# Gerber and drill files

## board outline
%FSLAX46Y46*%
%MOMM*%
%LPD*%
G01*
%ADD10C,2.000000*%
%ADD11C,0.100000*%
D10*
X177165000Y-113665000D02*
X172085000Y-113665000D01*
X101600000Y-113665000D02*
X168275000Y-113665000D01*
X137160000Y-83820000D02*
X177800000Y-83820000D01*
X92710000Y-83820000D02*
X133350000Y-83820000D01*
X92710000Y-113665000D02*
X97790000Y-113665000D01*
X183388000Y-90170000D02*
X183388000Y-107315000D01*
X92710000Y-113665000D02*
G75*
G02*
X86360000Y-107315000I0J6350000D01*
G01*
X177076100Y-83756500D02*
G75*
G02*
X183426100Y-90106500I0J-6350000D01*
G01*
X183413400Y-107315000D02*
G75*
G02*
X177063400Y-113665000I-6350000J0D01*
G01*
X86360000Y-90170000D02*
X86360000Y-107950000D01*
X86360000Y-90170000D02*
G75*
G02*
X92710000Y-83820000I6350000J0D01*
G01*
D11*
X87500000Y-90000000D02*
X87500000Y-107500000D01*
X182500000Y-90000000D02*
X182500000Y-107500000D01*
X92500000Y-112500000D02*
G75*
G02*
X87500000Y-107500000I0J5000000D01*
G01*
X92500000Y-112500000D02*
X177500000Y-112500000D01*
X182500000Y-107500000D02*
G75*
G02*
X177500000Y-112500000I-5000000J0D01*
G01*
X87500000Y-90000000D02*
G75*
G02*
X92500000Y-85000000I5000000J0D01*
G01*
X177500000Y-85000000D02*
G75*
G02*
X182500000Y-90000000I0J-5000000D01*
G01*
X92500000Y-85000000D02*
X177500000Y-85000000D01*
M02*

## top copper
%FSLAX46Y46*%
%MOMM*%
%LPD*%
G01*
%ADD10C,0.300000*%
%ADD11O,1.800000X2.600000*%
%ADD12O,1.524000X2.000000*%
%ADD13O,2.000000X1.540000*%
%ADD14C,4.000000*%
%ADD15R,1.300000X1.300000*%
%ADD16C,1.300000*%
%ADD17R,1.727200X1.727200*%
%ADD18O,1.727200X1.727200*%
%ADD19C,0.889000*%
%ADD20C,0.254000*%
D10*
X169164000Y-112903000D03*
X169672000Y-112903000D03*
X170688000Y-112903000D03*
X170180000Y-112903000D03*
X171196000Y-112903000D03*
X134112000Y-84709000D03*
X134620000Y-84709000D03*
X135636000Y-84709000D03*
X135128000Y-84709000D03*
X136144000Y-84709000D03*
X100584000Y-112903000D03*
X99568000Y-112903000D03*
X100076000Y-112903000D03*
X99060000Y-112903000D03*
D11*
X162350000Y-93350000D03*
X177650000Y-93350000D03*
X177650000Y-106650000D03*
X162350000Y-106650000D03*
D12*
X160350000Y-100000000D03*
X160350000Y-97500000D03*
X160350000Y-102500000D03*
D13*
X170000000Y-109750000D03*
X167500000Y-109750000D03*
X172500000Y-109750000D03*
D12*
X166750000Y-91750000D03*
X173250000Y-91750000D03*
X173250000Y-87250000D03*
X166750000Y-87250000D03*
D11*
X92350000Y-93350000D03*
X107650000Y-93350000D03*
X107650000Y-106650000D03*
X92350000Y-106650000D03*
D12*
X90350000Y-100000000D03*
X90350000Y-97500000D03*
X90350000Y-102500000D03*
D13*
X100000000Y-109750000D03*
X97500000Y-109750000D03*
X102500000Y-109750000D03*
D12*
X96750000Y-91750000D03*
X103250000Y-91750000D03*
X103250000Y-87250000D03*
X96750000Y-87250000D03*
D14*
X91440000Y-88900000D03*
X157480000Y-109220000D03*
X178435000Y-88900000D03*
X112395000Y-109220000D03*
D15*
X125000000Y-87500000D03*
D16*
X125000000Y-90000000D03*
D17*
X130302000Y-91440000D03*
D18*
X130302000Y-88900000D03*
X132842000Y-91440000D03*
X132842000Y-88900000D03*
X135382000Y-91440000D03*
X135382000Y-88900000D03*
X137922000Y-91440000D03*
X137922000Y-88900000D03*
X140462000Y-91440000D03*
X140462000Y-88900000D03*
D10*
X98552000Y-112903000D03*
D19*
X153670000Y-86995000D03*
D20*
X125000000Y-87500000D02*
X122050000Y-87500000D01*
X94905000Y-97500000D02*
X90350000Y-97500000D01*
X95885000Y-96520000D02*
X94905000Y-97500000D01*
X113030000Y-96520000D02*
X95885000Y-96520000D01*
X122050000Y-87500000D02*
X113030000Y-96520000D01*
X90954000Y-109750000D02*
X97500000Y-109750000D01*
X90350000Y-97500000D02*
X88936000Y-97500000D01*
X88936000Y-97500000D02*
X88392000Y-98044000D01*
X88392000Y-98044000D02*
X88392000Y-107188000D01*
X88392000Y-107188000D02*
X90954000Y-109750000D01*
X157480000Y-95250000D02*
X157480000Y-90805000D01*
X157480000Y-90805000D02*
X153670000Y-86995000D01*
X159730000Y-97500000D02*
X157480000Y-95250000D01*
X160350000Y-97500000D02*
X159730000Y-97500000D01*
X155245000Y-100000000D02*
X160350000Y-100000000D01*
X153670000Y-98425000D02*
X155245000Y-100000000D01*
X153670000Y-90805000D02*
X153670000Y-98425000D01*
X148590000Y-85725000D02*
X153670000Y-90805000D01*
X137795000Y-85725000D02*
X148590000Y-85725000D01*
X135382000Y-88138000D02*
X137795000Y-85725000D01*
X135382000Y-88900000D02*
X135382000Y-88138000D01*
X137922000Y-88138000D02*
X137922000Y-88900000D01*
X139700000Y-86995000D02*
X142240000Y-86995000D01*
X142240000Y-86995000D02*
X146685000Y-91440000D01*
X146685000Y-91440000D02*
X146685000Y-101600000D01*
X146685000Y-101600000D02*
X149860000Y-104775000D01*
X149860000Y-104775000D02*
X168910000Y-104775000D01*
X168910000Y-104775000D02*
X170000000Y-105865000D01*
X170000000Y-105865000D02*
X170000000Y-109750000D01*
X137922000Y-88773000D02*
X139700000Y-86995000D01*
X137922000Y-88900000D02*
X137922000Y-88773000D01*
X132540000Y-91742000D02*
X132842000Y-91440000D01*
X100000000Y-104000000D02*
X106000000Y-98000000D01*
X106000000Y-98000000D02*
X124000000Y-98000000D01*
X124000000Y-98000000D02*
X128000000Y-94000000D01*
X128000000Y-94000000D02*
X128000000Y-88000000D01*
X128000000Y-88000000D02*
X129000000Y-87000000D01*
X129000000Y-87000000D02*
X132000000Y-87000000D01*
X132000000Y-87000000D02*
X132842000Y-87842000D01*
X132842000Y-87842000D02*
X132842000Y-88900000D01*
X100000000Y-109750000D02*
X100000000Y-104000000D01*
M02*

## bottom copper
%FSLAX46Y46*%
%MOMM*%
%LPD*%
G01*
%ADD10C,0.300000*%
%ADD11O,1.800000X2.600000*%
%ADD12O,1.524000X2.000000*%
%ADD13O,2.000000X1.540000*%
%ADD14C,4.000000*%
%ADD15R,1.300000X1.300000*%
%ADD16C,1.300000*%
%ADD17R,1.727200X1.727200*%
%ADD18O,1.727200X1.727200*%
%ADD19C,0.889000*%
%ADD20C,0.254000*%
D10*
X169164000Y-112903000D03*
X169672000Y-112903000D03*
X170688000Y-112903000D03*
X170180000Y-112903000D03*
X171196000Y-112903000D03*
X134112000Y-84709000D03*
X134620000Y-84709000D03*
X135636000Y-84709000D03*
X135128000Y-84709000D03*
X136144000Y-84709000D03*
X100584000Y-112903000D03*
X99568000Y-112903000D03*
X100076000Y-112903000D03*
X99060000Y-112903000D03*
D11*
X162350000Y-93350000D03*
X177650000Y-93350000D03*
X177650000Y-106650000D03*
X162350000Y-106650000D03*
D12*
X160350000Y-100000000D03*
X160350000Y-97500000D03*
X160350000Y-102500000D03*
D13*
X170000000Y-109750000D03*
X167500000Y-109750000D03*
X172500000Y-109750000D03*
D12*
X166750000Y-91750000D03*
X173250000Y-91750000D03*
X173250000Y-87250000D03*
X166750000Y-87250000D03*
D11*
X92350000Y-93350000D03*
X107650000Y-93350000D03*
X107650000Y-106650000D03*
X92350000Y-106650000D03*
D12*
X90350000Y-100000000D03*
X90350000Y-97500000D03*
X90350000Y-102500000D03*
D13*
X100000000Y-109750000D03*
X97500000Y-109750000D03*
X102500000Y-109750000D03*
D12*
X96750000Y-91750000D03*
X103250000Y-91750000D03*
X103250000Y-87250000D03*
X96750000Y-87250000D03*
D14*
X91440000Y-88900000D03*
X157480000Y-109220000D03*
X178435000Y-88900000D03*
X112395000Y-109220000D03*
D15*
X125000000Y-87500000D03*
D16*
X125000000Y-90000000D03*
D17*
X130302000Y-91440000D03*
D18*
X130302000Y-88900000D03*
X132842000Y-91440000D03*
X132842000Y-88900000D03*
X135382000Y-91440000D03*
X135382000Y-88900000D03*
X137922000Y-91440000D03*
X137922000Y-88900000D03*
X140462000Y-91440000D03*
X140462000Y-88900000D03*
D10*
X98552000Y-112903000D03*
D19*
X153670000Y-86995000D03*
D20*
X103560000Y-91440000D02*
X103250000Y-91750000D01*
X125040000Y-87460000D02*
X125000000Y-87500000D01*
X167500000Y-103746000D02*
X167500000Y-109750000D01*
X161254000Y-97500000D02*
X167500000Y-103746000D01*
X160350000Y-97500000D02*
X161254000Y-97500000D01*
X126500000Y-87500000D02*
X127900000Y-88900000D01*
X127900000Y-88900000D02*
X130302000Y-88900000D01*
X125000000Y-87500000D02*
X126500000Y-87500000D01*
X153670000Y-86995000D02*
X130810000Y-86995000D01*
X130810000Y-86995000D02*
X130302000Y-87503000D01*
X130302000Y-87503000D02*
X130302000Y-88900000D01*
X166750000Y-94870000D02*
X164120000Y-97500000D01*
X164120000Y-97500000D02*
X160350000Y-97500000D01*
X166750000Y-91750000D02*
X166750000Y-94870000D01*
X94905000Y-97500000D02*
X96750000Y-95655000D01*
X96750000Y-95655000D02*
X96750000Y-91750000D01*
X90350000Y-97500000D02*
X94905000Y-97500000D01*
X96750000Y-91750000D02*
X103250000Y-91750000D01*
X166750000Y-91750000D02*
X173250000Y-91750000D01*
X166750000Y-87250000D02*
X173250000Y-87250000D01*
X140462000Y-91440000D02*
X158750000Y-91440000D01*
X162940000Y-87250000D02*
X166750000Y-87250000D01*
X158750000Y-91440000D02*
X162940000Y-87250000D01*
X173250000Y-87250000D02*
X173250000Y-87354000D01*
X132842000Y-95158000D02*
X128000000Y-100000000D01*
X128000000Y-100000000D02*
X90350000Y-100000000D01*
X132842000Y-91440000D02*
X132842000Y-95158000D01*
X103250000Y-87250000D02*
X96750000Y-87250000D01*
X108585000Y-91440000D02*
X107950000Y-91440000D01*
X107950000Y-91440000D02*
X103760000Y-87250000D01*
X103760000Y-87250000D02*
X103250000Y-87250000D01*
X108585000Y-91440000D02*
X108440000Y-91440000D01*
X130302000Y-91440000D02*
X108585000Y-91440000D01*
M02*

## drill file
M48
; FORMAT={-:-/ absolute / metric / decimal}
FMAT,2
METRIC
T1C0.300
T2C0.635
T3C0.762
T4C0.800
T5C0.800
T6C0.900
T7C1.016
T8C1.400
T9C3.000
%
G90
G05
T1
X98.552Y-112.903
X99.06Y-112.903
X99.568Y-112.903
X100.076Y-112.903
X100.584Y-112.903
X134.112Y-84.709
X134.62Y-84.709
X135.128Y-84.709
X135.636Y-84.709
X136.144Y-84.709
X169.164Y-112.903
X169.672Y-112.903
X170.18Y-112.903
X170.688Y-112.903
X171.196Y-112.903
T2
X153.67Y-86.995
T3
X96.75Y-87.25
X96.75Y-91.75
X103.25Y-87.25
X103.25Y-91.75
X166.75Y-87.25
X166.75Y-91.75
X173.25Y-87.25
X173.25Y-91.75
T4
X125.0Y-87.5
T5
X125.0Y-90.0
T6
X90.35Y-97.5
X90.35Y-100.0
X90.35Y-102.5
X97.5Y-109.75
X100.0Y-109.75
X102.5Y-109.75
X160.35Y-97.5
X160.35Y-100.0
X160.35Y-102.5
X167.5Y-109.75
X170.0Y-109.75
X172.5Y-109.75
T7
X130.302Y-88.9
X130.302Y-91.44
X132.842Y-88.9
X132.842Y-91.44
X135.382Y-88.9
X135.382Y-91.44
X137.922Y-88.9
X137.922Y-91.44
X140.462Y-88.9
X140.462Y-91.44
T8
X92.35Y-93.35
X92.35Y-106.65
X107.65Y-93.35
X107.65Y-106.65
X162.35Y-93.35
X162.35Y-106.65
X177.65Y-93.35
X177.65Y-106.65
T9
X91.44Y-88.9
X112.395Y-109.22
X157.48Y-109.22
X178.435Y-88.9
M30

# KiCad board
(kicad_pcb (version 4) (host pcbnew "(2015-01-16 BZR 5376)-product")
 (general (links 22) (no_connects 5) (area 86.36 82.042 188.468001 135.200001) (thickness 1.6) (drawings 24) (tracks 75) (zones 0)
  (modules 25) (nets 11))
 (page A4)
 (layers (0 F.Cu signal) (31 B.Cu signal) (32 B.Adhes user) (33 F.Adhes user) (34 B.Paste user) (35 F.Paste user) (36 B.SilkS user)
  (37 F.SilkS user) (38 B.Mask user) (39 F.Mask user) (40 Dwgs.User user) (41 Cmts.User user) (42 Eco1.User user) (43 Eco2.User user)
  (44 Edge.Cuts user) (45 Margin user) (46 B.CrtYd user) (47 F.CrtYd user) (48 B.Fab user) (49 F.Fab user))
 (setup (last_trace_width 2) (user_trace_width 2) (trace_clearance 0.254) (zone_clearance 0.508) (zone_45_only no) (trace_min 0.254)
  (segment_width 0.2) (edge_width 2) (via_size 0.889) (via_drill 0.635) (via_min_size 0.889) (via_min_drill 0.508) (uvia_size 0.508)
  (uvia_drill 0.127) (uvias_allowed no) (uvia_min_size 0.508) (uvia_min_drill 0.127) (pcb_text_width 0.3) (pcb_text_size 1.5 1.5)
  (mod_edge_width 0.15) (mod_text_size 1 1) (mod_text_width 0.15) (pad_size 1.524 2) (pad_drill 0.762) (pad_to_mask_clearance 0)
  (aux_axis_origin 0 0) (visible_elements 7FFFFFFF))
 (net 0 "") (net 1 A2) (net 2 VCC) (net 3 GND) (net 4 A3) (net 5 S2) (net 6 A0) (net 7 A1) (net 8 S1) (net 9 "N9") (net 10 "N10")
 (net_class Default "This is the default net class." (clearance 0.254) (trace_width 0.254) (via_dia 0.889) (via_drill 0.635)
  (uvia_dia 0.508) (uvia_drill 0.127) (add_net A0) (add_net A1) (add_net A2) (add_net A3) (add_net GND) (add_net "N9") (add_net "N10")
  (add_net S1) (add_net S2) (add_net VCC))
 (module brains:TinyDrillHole (layer F.Cu) (at 169.164 112.903)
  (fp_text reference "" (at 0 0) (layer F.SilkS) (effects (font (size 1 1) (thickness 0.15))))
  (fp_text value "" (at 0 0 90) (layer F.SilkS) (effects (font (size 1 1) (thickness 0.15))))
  (pad 2 thru_hole circle (at 0 0) (size 0.3 0.3) (drill 0.3) (layers *.Cu *.Mask F.SilkS)))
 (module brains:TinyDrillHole (layer F.Cu) (at 169.672 112.903)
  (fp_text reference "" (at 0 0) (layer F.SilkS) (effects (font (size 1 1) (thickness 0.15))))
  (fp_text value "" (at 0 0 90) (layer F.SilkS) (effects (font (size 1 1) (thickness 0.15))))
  (pad 2 thru_hole circle (at 0 0) (size 0.3 0.3) (drill 0.3) (layers *.Cu *.Mask F.SilkS)))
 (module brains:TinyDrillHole (layer F.Cu) (at 170.688 112.903)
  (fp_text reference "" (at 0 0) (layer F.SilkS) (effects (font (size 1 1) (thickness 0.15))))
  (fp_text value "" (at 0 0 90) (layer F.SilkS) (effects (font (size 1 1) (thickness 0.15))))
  (pad 2 thru_hole circle (at 0 0) (size 0.3 0.3) (drill 0.3) (layers *.Cu *.Mask F.SilkS)))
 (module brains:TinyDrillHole (layer F.Cu) (at 170.18 112.903)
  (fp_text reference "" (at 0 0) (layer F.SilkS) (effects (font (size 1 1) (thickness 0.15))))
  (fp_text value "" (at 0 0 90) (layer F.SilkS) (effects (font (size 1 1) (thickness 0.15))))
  (pad 2 thru_hole circle (at 0 0) (size 0.3 0.3) (drill 0.3) (layers *.Cu *.Mask F.SilkS)))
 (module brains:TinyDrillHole (layer F.Cu) (at 171.196 112.903)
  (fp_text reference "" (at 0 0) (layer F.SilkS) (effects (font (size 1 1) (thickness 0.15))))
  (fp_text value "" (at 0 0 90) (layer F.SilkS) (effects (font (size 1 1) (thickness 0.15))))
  (pad 2 thru_hole circle (at 0 0) (size 0.3 0.3) (drill 0.3) (layers *.Cu *.Mask F.SilkS)))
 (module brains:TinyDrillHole (layer F.Cu) (at 134.112 84.709)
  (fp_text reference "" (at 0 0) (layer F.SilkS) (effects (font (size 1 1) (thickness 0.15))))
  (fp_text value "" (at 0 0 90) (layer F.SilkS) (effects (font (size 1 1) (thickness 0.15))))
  (pad 2 thru_hole circle (at 0 0) (size 0.3 0.3) (drill 0.3) (layers *.Cu *.Mask F.SilkS)))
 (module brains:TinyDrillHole (layer F.Cu) (at 134.62 84.709)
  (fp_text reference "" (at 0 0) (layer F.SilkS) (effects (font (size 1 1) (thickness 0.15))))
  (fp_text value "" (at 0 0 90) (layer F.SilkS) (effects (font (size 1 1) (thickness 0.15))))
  (pad 2 thru_hole circle (at 0 0) (size 0.3 0.3) (drill 0.3) (layers *.Cu *.Mask F.SilkS)))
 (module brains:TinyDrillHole (layer F.Cu) (at 135.636 84.709)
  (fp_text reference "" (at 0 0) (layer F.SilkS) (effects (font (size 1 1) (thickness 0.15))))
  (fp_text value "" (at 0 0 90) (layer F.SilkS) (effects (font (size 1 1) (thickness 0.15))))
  (pad 2 thru_hole circle (at 0 0) (size 0.3 0.3) (drill 0.3) (layers *.Cu *.Mask F.SilkS)))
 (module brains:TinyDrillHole (layer F.Cu) (at 135.128 84.709)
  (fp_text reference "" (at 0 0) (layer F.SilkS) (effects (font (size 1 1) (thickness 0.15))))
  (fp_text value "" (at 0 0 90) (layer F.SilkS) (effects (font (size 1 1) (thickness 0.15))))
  (pad 2 thru_hole circle (at 0 0) (size 0.3 0.3) (drill 0.3) (layers *.Cu *.Mask F.SilkS)))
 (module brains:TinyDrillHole (layer F.Cu) (at 136.144 84.709)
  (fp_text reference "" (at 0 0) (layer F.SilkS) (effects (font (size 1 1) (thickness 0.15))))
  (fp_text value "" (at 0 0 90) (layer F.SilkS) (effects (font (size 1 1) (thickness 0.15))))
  (pad 2 thru_hole circle (at 0 0) (size 0.3 0.3) (drill 0.3) (layers *.Cu *.Mask F.SilkS)))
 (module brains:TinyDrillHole (layer F.Cu) (at 100.584 112.903)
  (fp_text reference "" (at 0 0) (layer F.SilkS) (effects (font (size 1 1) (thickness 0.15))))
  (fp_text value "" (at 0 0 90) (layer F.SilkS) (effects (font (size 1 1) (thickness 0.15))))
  (pad 2 thru_hole circle (at 0 0) (size 0.3 0.3) (drill 0.3) (layers *.Cu *.Mask F.SilkS)))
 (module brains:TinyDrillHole (layer F.Cu) (at 99.568 112.903)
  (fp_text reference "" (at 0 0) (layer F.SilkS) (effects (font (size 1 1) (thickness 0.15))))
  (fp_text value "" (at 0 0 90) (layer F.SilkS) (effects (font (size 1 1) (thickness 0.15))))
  (pad 2 thru_hole circle (at 0 0) (size 0.3 0.3) (drill 0.3) (layers *.Cu *.Mask F.SilkS)))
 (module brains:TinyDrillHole (layer F.Cu) (at 100.076 112.903)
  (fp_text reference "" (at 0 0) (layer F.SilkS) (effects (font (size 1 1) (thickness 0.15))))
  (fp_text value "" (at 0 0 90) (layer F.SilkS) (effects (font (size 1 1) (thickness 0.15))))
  (pad 2 thru_hole circle (at 0 0) (size 0.3 0.3) (drill 0.3) (layers *.Cu *.Mask F.SilkS)))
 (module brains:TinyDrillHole (layer F.Cu) (at 99.06 112.903)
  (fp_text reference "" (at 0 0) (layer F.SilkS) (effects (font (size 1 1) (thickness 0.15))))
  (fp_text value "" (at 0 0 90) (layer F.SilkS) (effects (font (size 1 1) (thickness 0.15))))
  (pad 2 thru_hole circle (at 0 0) (size 0.3 0.3) (drill 0.3) (layers *.Cu *.Mask F.SilkS)))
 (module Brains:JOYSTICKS (layer F.Cu) (at 170 100)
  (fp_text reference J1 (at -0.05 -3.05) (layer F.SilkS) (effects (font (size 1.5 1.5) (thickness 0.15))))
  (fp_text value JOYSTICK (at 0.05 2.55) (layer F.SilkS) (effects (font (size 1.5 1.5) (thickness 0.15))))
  (pad "" thru_hole oval (at -7.65 -6.65) (size 1.8 2.6) (drill 1.4) (layers *.Cu *.Mask F.SilkS))
  (pad "" thru_hole oval (at 7.65 -6.65) (size 1.8 2.6) (drill 1.4) (layers *.Cu *.Mask F.SilkS))
  (pad "" thru_hole oval (at 7.65 6.65) (size 1.8 2.6) (drill 1.4) (layers *.Cu *.Mask F.SilkS))
  (pad "" thru_hole oval (at -7.65 6.65) (size 1.8 2.6) (drill 1.4) (layers *.Cu *.Mask F.SilkS))
  (pad 4 thru_hole oval (at -9.65 0) (size 1.524 2) (drill 0.9) (layers *.Cu *.Mask F.SilkS) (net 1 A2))
  (pad 3 thru_hole oval (at -9.65 -2.5) (size 1.524 2) (drill 0.9) (layers *.Cu *.Mask F.SilkS) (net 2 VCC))
  (pad 5 thru_hole oval (at -9.65 2.5) (size 1.524 2) (drill 0.9) (layers *.Cu *.Mask F.SilkS) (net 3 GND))
  (pad 7 thru_hole oval (at 0 9.75) (size 2 1.54) (drill 0.9) (layers *.Cu *.Mask F.SilkS) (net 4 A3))
  (pad 6 thru_hole oval (at -2.5 9.75) (size 2 1.54) (drill 0.9) (layers *.Cu *.Mask F.SilkS) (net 2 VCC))
  (pad 8 thru_hole oval (at 2.5 9.75) (size 2 1.54) (drill 0.9) (layers *.Cu *.Mask F.SilkS) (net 3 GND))
  (pad 2 thru_hole oval (at -3.25 -8.25) (size 1.524 2) (drill 0.762) (layers *.Cu *.Mask F.SilkS) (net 2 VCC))
  (pad 2 thru_hole oval (at 3.25 -8.25) (size 1.524 2) (drill 0.762) (layers *.Cu *.Mask F.SilkS) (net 2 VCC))
  (pad 1 thru_hole oval (at 3.25 -12.75) (size 1.524 2) (drill 0.762) (layers *.Cu *.Mask F.SilkS) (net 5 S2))
  (pad 1 thru_hole oval (at -3.25 -12.75) (size 1.524 2) (drill 0.762) (layers *.Cu *.Mask F.SilkS) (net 5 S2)))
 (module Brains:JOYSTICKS (layer F.Cu) (at 100 100)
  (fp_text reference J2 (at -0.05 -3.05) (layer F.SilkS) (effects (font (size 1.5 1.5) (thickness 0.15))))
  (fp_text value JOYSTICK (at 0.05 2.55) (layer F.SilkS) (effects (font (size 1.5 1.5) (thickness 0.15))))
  (pad "" thru_hole oval (at -7.65 -6.65) (size 1.8 2.6) (drill 1.4) (layers *.Cu *.Mask F.SilkS))
  (pad "" thru_hole oval (at 7.65 -6.65) (size 1.8 2.6) (drill 1.4) (layers *.Cu *.Mask F.SilkS))
  (pad "" thru_hole oval (at 7.65 6.65) (size 1.8 2.6) (drill 1.4) (layers *.Cu *.Mask F.SilkS))
  (pad "" thru_hole oval (at -7.65 6.65) (size 1.8 2.6) (drill 1.4) (layers *.Cu *.Mask F.SilkS))
  (pad 4 thru_hole oval (at -9.65 0) (size 1.524 2) (drill 0.9) (layers *.Cu *.Mask F.SilkS) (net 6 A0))
  (pad 3 thru_hole oval (at -9.65 -2.5) (size 1.524 2) (drill 0.9) (layers *.Cu *.Mask F.SilkS) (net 2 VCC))
  (pad 5 thru_hole oval (at -9.65 2.5) (size 1.524 2) (drill 0.9) (layers *.Cu *.Mask F.SilkS) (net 3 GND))
  (pad 7 thru_hole oval (at 0 9.75) (size 2 1.54) (drill 0.9) (layers *.Cu *.Mask F.SilkS) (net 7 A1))
  (pad 6 thru_hole oval (at -2.5 9.75) (size 2 1.54) (drill 0.9) (layers *.Cu *.Mask F.SilkS) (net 2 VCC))
  (pad 8 thru_hole oval (at 2.5 9.75) (size 2 1.54) (drill 0.9) (layers *.Cu *.Mask F.SilkS) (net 3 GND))
  (pad 2 thru_hole oval (at -3.25 -8.25) (size 1.524 2) (drill 0.762) (layers *.Cu *.Mask F.SilkS) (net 2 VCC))
  (pad 2 thru_hole oval (at 3.25 -8.25) (size 1.524 2) (drill 0.762) (layers *.Cu *.Mask F.SilkS) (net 2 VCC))
  (pad 1 thru_hole oval (at 3.25 -12.75) (size 1.524 2) (drill 0.762) (layers *.Cu *.Mask F.SilkS) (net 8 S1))
  (pad 1 thru_hole oval (at -3.25 -12.75) (size 1.524 2) (drill 0.762) (layers *.Cu *.Mask F.SilkS) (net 8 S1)))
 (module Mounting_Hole (layer F.Cu) (at 91.44 88.9)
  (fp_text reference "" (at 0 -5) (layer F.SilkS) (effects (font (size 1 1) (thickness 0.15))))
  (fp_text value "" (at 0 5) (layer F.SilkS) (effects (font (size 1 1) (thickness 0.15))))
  (pad "" thru_hole circle (at 0 0) (size 4 4) (drill 3) (layers *.Cu *.Mask F.SilkS)))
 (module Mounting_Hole (layer F.Cu) (at 157.48 109.22)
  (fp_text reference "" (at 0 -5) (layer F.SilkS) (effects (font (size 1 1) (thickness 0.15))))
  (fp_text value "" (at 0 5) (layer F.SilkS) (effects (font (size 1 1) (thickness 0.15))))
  (pad "" thru_hole circle (at 0 0) (size 4 4) (drill 3) (layers *.Cu *.Mask F.SilkS)))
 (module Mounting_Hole (layer F.Cu) (at 178.435 88.9)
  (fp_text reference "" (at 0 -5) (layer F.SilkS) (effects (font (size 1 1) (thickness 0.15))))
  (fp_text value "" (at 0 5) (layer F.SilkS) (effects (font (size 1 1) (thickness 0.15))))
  (pad "" thru_hole circle (at 0 0) (size 4 4) (drill 3) (layers *.Cu *.Mask F.SilkS)))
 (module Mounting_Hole (layer F.Cu) (at 112.395 109.22)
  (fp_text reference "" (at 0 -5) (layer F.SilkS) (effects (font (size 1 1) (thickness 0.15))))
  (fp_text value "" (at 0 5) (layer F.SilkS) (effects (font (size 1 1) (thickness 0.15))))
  (pad "" thru_hole circle (at 0 0) (size 4 4) (drill 3) (layers *.Cu *.Mask F.SilkS)))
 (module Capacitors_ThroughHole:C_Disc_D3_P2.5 (layer F.Cu) (at 125 87.5 270)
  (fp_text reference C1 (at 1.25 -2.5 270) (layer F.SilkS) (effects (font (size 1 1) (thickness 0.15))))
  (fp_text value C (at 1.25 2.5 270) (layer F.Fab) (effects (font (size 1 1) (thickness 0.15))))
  (pad 1 thru_hole rect (at 0 0 270) (size 1.3 1.3) (drill 0.8) (layers *.Cu *.Mask F.SilkS) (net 2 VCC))
  (pad 2 thru_hole circle (at 2.5 0 270) (size 1.3 1.3) (drill 0.8001) (layers *.Cu *.Mask F.SilkS) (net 3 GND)))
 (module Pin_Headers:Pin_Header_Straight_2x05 (layer F.Cu) (at 130.302 91.44 90)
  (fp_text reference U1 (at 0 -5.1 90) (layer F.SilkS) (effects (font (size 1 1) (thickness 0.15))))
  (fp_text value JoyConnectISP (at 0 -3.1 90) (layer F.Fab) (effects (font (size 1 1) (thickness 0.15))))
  (pad 1 thru_hole rect (at 0 0 90) (size 1.7272 1.7272) (drill 1.016) (layers *.Cu *.Mask F.SilkS) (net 8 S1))
  (pad 2 thru_hole oval (at 2.54 0 90) (size 1.7272 1.7272) (drill 1.016) (layers *.Cu *.Mask F.SilkS) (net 2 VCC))
  (pad 3 thru_hole oval (at 0 2.54 90) (size 1.7272 1.7272) (drill 1.016) (layers *.Cu *.Mask F.SilkS) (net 6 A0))
  (pad 4 thru_hole oval (at 2.54 2.54 90) (size 1.7272 1.7272) (drill 1.016) (layers *.Cu *.Mask F.SilkS) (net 7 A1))
  (pad 5 thru_hole oval (at 0 5.08 90) (size 1.7272 1.7272) (drill 1.016) (layers *.Cu *.Mask F.SilkS) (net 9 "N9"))
  (pad 6 thru_hole oval (at 2.54 5.08 90) (size 1.7272 1.7272) (drill 1.016) (layers *.Cu *.Mask F.SilkS) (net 1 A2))
  (pad 7 thru_hole oval (at 0 7.62 90) (size 1.7272 1.7272) (drill 1.016) (layers *.Cu *.Mask F.SilkS) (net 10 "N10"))
  (pad 8 thru_hole oval (at 2.54 7.62 90) (size 1.7272 1.7272) (drill 1.016) (layers *.Cu *.Mask F.SilkS) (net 4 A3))
  (pad 9 thru_hole oval (at 0 10.16 90) (size 1.7272 1.7272) (drill 1.016) (layers *.Cu *.Mask F.SilkS) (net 5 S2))
  (pad 10 thru_hole oval (at 2.54 10.16 90) (size 1.7272 1.7272) (drill 1.016) (layers *.Cu *.Mask F.SilkS) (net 3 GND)))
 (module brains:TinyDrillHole (layer F.Cu) (at 98.552 112.903)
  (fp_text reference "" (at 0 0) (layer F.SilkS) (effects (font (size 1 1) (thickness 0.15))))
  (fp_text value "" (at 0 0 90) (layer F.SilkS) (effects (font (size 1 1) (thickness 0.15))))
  (pad 2 thru_hole circle (at 0 0) (size 0.3 0.3) (drill 0.3) (layers *.Cu *.Mask F.SilkS)))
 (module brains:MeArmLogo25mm (layer B.Cu) (at 143.764 99.187 180)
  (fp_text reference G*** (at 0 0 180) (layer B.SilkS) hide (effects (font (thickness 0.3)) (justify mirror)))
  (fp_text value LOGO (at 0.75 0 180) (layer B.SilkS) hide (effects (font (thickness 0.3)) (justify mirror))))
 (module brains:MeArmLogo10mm (layer F.Cu) (at 117.856 98.171)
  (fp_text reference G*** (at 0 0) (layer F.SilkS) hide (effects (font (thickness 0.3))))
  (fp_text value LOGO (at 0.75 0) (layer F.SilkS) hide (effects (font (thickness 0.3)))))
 (gr_line (start 177.165 113.665) (end 172.085 113.665) (angle 90) (layer Edge.Cuts) (width 2))
 (gr_line (start 101.6 113.665) (end 168.275 113.665) (angle 90) (layer Edge.Cuts) (width 2))
 (gr_line (start 137.16 83.82) (end 177.8 83.82) (angle 90) (layer Edge.Cuts) (width 2))
 (gr_line (start 92.71 83.82) (end 133.35 83.82) (angle 90) (layer Edge.Cuts) (width 2))
 (gr_line (start 92.71 113.665) (end 97.79 113.665) (angle 90) (layer Edge.Cuts) (width 2))
 (gr_line (start 183.388 90.17) (end 183.388 107.315) (angle 90) (layer Edge.Cuts) (width 2))
 (gr_arc (start 92.71 107.315) (end 86.36 107.315) (angle -90) (layer Edge.Cuts) (width 2))
 (gr_arc (start 177.0761 90.1065) (end 183.4261 90.1065) (angle -90) (layer Edge.Cuts) (width 2))
 (gr_arc (start 177.0634 107.315) (end 183.4134 107.315) (angle 90) (layer Edge.Cuts) (width 2))
 (gr_line (start 86.36 90.17) (end 86.36 107.95) (angle 90) (layer Edge.Cuts) (width 2))
 (gr_arc (start 92.71 90.17) (end 86.36 90.17) (angle 90) (layer Edge.Cuts) (width 2))
 (gr_line (start 87.5 90) (end 87.5 107.5) (angle 90) (layer Edge.Cuts) (width 0.1))
 (gr_line (start 182.5 90) (end 182.5 107.5) (angle 90) (layer Edge.Cuts) (width 0.1))
 (gr_arc (start 92.5 107.5) (end 92.5 112.5) (angle 90) (layer Edge.Cuts) (width 0.1))
 (gr_line (start 92.5 112.5) (end 177.5 112.5) (angle 90) (layer Edge.Cuts) (width 0.1))
 (gr_arc (start 177.5 107.5) (end 182.5 107.5) (angle 90) (layer Edge.Cuts) (width 0.1))
 (gr_arc (start 92.5 90) (end 87.5 90) (angle 90) (layer Edge.Cuts) (width 0.1))
 (gr_arc (start 177.5 90) (end 177.5 85) (angle 90) (layer Edge.Cuts) (width 0.1))
 (gr_line (start 92.5 85) (end 177.5 85) (angle 90) (layer Edge.Cuts) (width 0.1))
 (segment (start 103.56 91.44) (end 103.25 91.75) (width 0.254) (layer B.Cu) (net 2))
 (segment (start 125 87.5) (end 122.05 87.5) (width 0.254) (layer F.Cu) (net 2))
 (segment (start 94.905 97.5) (end 90.35 97.5) (width 0.254) (layer F.Cu) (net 2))
 (segment (start 95.885 96.52) (end 94.905 97.5) (width 0.254) (layer F.Cu) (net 2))
 (segment (start 113.03 96.52) (end 95.885 96.52) (width 0.254) (layer F.Cu) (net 2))
 (segment (start 122.05 87.5) (end 113.03 96.52) (width 0.254) (layer F.Cu) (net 2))
 (segment (start 125.04 87.46) (end 125 87.5) (width 0.254) (layer B.Cu) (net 2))
 (segment (start 90.954 109.75) (end 97.5 109.75) (width 0.254) (layer F.Cu) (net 2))
 (segment (start 90.35 97.5) (end 88.936 97.5) (width 0.254) (layer F.Cu) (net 2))
 (segment (start 88.936 97.5) (end 88.392 98.044) (width 0.254) (layer F.Cu) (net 2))
 (segment (start 88.392 98.044) (end 88.392 107.188) (width 0.254) (layer F.Cu) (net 2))
 (segment (start 88.392 107.188) (end 90.954 109.75) (width 0.254) (layer F.Cu) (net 2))
 (segment (start 167.5 103.746) (end 167.5 109.75) (width 0.254) (layer B.Cu) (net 2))
 (segment (start 161.254 97.5) (end 167.5 103.746) (width 0.254) (layer B.Cu) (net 2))
 (segment (start 160.35 97.5) (end 161.254 97.5) (width 0.254) (layer B.Cu) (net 2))
 (segment (start 126.5 87.5) (end 127.9 88.9) (width 0.254) (layer B.Cu) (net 2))
 (segment (start 127.9 88.9) (end 130.302 88.9) (width 0.254) (layer B.Cu) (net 2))
 (segment (start 125 87.5) (end 126.5 87.5) (width 0.254) (layer B.Cu) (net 2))
 (segment (start 157.48 95.25) (end 157.48 90.805) (width 0.254) (layer F.Cu) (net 2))
 (segment (start 157.48 90.805) (end 153.67 86.995) (width 0.254) (layer F.Cu) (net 2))
 (via (at 153.67 86.995) (size 0.889) (layers F.Cu B.Cu) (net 2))
 (segment (start 153.67 86.995) (end 130.81 86.995) (width 0.254) (layer B.Cu) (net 2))
 (segment (start 130.81 86.995) (end 130.302 87.503) (width 0.254) (layer B.Cu) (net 2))
 (segment (start 130.302 87.503) (end 130.302 88.9) (width 0.254) (layer B.Cu) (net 2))
 (segment (start 159.73 97.5) (end 157.48 95.25) (width 0.254) (layer F.Cu) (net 2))
 (segment (start 160.35 97.5) (end 159.73 97.5) (width 0.254) (layer F.Cu) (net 2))
 (segment (start 166.75 94.87) (end 164.12 97.5) (width 0.254) (layer B.Cu) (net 2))
 (segment (start 164.12 97.5) (end 160.35 97.5) (width 0.254) (layer B.Cu) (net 2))
 (segment (start 166.75 91.75) (end 166.75 94.87) (width 0.254) (layer B.Cu) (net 2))
 (segment (start 94.905 97.5) (end 96.75 95.655) (width 0.254) (layer B.Cu) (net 2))
 (segment (start 96.75 95.655) (end 96.75 91.75) (width 0.254) (layer B.Cu) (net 2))
 (segment (start 90.35 97.5) (end 94.905 97.5) (width 0.254) (layer B.Cu) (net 2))
 (segment (start 96.75 91.75) (end 103.25 91.75) (width 0.254) (layer B.Cu) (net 2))
 (segment (start 166.75 91.75) (end 173.25 91.75) (width 0.254) (layer B.Cu) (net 2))
 (segment (start 155.245 100) (end 160.35 100) (width 0.254) (layer F.Cu) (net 1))
 (segment (start 153.67 98.425) (end 155.245 100) (width 0.254) (layer F.Cu) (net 1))
 (segment (start 153.67 90.805) (end 153.67 98.425) (width 0.254) (layer F.Cu) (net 1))
 (segment (start 148.59 85.725) (end 153.67 90.805) (width 0.254) (layer F.Cu) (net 1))
 (segment (start 137.795 85.725) (end 148.59 85.725) (width 0.254) (layer F.Cu) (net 1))
 (segment (start 135.382 88.138) (end 137.795 85.725) (width 0.254) (layer F.Cu) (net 1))
 (segment (start 135.382 88.9) (end 135.382 88.138) (width 0.254) (layer F.Cu) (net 1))
 (segment (start 137.922 88.138) (end 137.922 88.9) (width 0.254) (layer F.Cu) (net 4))
 (segment (start 139.7 86.995) (end 142.24 86.995) (width 0.254) (layer F.Cu) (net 4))
 (segment (start 142.24 86.995) (end 146.685 91.44) (width 0.254) (layer F.Cu) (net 4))
 (segment (start 146.685 91.44) (end 146.685 101.6) (width 0.254) (layer F.Cu) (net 4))
 (segment (start 146.685 101.6) (end 149.86 104.775) (width 0.254) (layer F.Cu) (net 4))
 (segment (start 149.86 104.775) (end 168.91 104.775) (width 0.254) (layer F.Cu) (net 4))
 (segment (start 168.91 104.775) (end 170 105.865) (width 0.254) (layer F.Cu) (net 4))
 (segment (start 170 105.865) (end 170 109.75) (width 0.254) (layer F.Cu) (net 4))
 (segment (start 137.922 88.773) (end 139.7 86.995) (width 0.254) (layer F.Cu) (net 4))
 (segment (start 137.922 88.9) (end 137.922 88.773) (width 0.254) (layer F.Cu) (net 4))
 (segment (start 166.75 87.25) (end 173.25 87.25) (width 0.254) (layer B.Cu) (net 5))
 (segment (start 140.462 91.44) (end 158.75 91.44) (width 0.254) (layer B.Cu) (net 5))
 (segment (start 162.94 87.25) (end 166.75 87.25) (width 0.254) (layer B.Cu) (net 5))
 (segment (start 158.75 91.44) (end 162.94 87.25) (width 0.254) (layer B.Cu) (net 5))
 (segment (start 173.25 87.25) (end 173.25 87.354) (width 0.254) (layer B.Cu) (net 5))
 (segment (start 132.54 91.742) (end 132.842 91.44) (width 0.254) (layer F.Cu) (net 6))
 (segment (start 132.842 95.158) (end 128 100) (width 0.254) (layer B.Cu) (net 6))
 (segment (start 128 100) (end 90.35 100) (width 0.254) (layer B.Cu) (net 6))
 (segment (start 132.842 91.44) (end 132.842 95.158) (width 0.254) (layer B.Cu) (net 6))
 (segment (start 100 104) (end 106 98) (width 0.254) (layer F.Cu) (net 7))
 (segment (start 106 98) (end 124 98) (width 0.254) (layer F.Cu) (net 7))
 (segment (start 124 98) (end 128 94) (width 0.254) (layer F.Cu) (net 7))
 (segment (start 128 94) (end 128 88) (width 0.254) (layer F.Cu) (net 7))
 (segment (start 128 88) (end 129 87) (width 0.254) (layer F.Cu) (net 7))
 (segment (start 129 87) (end 132 87) (width 0.254) (layer F.Cu) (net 7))
 (segment (start 132 87) (end 132.842 87.842) (width 0.254) (layer F.Cu) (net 7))
 (segment (start 132.842 87.842) (end 132.842 88.9) (width 0.254) (layer F.Cu) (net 7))
 (segment (start 100 109.75) (end 100 104) (width 0.254) (layer F.Cu) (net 7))
 (segment (start 103.25 87.25) (end 96.75 87.25) (width 0.254) (layer B.Cu) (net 8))
 (segment (start 108.585 91.44) (end 107.95 91.44) (width 0.254) (layer B.Cu) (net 8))
 (segment (start 107.95 91.44) (end 103.76 87.25) (width 0.254) (layer B.Cu) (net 8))
 (segment (start 103.76 87.25) (end 103.25 87.25) (width 0.254) (layer B.Cu) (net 8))
 (segment (start 108.585 91.44) (end 108.44 91.44) (width 0.254) (layer B.Cu) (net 8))
 (segment (start 130.302 91.44) (end 108.585 91.44) (width 0.254) (layer B.Cu) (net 8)))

